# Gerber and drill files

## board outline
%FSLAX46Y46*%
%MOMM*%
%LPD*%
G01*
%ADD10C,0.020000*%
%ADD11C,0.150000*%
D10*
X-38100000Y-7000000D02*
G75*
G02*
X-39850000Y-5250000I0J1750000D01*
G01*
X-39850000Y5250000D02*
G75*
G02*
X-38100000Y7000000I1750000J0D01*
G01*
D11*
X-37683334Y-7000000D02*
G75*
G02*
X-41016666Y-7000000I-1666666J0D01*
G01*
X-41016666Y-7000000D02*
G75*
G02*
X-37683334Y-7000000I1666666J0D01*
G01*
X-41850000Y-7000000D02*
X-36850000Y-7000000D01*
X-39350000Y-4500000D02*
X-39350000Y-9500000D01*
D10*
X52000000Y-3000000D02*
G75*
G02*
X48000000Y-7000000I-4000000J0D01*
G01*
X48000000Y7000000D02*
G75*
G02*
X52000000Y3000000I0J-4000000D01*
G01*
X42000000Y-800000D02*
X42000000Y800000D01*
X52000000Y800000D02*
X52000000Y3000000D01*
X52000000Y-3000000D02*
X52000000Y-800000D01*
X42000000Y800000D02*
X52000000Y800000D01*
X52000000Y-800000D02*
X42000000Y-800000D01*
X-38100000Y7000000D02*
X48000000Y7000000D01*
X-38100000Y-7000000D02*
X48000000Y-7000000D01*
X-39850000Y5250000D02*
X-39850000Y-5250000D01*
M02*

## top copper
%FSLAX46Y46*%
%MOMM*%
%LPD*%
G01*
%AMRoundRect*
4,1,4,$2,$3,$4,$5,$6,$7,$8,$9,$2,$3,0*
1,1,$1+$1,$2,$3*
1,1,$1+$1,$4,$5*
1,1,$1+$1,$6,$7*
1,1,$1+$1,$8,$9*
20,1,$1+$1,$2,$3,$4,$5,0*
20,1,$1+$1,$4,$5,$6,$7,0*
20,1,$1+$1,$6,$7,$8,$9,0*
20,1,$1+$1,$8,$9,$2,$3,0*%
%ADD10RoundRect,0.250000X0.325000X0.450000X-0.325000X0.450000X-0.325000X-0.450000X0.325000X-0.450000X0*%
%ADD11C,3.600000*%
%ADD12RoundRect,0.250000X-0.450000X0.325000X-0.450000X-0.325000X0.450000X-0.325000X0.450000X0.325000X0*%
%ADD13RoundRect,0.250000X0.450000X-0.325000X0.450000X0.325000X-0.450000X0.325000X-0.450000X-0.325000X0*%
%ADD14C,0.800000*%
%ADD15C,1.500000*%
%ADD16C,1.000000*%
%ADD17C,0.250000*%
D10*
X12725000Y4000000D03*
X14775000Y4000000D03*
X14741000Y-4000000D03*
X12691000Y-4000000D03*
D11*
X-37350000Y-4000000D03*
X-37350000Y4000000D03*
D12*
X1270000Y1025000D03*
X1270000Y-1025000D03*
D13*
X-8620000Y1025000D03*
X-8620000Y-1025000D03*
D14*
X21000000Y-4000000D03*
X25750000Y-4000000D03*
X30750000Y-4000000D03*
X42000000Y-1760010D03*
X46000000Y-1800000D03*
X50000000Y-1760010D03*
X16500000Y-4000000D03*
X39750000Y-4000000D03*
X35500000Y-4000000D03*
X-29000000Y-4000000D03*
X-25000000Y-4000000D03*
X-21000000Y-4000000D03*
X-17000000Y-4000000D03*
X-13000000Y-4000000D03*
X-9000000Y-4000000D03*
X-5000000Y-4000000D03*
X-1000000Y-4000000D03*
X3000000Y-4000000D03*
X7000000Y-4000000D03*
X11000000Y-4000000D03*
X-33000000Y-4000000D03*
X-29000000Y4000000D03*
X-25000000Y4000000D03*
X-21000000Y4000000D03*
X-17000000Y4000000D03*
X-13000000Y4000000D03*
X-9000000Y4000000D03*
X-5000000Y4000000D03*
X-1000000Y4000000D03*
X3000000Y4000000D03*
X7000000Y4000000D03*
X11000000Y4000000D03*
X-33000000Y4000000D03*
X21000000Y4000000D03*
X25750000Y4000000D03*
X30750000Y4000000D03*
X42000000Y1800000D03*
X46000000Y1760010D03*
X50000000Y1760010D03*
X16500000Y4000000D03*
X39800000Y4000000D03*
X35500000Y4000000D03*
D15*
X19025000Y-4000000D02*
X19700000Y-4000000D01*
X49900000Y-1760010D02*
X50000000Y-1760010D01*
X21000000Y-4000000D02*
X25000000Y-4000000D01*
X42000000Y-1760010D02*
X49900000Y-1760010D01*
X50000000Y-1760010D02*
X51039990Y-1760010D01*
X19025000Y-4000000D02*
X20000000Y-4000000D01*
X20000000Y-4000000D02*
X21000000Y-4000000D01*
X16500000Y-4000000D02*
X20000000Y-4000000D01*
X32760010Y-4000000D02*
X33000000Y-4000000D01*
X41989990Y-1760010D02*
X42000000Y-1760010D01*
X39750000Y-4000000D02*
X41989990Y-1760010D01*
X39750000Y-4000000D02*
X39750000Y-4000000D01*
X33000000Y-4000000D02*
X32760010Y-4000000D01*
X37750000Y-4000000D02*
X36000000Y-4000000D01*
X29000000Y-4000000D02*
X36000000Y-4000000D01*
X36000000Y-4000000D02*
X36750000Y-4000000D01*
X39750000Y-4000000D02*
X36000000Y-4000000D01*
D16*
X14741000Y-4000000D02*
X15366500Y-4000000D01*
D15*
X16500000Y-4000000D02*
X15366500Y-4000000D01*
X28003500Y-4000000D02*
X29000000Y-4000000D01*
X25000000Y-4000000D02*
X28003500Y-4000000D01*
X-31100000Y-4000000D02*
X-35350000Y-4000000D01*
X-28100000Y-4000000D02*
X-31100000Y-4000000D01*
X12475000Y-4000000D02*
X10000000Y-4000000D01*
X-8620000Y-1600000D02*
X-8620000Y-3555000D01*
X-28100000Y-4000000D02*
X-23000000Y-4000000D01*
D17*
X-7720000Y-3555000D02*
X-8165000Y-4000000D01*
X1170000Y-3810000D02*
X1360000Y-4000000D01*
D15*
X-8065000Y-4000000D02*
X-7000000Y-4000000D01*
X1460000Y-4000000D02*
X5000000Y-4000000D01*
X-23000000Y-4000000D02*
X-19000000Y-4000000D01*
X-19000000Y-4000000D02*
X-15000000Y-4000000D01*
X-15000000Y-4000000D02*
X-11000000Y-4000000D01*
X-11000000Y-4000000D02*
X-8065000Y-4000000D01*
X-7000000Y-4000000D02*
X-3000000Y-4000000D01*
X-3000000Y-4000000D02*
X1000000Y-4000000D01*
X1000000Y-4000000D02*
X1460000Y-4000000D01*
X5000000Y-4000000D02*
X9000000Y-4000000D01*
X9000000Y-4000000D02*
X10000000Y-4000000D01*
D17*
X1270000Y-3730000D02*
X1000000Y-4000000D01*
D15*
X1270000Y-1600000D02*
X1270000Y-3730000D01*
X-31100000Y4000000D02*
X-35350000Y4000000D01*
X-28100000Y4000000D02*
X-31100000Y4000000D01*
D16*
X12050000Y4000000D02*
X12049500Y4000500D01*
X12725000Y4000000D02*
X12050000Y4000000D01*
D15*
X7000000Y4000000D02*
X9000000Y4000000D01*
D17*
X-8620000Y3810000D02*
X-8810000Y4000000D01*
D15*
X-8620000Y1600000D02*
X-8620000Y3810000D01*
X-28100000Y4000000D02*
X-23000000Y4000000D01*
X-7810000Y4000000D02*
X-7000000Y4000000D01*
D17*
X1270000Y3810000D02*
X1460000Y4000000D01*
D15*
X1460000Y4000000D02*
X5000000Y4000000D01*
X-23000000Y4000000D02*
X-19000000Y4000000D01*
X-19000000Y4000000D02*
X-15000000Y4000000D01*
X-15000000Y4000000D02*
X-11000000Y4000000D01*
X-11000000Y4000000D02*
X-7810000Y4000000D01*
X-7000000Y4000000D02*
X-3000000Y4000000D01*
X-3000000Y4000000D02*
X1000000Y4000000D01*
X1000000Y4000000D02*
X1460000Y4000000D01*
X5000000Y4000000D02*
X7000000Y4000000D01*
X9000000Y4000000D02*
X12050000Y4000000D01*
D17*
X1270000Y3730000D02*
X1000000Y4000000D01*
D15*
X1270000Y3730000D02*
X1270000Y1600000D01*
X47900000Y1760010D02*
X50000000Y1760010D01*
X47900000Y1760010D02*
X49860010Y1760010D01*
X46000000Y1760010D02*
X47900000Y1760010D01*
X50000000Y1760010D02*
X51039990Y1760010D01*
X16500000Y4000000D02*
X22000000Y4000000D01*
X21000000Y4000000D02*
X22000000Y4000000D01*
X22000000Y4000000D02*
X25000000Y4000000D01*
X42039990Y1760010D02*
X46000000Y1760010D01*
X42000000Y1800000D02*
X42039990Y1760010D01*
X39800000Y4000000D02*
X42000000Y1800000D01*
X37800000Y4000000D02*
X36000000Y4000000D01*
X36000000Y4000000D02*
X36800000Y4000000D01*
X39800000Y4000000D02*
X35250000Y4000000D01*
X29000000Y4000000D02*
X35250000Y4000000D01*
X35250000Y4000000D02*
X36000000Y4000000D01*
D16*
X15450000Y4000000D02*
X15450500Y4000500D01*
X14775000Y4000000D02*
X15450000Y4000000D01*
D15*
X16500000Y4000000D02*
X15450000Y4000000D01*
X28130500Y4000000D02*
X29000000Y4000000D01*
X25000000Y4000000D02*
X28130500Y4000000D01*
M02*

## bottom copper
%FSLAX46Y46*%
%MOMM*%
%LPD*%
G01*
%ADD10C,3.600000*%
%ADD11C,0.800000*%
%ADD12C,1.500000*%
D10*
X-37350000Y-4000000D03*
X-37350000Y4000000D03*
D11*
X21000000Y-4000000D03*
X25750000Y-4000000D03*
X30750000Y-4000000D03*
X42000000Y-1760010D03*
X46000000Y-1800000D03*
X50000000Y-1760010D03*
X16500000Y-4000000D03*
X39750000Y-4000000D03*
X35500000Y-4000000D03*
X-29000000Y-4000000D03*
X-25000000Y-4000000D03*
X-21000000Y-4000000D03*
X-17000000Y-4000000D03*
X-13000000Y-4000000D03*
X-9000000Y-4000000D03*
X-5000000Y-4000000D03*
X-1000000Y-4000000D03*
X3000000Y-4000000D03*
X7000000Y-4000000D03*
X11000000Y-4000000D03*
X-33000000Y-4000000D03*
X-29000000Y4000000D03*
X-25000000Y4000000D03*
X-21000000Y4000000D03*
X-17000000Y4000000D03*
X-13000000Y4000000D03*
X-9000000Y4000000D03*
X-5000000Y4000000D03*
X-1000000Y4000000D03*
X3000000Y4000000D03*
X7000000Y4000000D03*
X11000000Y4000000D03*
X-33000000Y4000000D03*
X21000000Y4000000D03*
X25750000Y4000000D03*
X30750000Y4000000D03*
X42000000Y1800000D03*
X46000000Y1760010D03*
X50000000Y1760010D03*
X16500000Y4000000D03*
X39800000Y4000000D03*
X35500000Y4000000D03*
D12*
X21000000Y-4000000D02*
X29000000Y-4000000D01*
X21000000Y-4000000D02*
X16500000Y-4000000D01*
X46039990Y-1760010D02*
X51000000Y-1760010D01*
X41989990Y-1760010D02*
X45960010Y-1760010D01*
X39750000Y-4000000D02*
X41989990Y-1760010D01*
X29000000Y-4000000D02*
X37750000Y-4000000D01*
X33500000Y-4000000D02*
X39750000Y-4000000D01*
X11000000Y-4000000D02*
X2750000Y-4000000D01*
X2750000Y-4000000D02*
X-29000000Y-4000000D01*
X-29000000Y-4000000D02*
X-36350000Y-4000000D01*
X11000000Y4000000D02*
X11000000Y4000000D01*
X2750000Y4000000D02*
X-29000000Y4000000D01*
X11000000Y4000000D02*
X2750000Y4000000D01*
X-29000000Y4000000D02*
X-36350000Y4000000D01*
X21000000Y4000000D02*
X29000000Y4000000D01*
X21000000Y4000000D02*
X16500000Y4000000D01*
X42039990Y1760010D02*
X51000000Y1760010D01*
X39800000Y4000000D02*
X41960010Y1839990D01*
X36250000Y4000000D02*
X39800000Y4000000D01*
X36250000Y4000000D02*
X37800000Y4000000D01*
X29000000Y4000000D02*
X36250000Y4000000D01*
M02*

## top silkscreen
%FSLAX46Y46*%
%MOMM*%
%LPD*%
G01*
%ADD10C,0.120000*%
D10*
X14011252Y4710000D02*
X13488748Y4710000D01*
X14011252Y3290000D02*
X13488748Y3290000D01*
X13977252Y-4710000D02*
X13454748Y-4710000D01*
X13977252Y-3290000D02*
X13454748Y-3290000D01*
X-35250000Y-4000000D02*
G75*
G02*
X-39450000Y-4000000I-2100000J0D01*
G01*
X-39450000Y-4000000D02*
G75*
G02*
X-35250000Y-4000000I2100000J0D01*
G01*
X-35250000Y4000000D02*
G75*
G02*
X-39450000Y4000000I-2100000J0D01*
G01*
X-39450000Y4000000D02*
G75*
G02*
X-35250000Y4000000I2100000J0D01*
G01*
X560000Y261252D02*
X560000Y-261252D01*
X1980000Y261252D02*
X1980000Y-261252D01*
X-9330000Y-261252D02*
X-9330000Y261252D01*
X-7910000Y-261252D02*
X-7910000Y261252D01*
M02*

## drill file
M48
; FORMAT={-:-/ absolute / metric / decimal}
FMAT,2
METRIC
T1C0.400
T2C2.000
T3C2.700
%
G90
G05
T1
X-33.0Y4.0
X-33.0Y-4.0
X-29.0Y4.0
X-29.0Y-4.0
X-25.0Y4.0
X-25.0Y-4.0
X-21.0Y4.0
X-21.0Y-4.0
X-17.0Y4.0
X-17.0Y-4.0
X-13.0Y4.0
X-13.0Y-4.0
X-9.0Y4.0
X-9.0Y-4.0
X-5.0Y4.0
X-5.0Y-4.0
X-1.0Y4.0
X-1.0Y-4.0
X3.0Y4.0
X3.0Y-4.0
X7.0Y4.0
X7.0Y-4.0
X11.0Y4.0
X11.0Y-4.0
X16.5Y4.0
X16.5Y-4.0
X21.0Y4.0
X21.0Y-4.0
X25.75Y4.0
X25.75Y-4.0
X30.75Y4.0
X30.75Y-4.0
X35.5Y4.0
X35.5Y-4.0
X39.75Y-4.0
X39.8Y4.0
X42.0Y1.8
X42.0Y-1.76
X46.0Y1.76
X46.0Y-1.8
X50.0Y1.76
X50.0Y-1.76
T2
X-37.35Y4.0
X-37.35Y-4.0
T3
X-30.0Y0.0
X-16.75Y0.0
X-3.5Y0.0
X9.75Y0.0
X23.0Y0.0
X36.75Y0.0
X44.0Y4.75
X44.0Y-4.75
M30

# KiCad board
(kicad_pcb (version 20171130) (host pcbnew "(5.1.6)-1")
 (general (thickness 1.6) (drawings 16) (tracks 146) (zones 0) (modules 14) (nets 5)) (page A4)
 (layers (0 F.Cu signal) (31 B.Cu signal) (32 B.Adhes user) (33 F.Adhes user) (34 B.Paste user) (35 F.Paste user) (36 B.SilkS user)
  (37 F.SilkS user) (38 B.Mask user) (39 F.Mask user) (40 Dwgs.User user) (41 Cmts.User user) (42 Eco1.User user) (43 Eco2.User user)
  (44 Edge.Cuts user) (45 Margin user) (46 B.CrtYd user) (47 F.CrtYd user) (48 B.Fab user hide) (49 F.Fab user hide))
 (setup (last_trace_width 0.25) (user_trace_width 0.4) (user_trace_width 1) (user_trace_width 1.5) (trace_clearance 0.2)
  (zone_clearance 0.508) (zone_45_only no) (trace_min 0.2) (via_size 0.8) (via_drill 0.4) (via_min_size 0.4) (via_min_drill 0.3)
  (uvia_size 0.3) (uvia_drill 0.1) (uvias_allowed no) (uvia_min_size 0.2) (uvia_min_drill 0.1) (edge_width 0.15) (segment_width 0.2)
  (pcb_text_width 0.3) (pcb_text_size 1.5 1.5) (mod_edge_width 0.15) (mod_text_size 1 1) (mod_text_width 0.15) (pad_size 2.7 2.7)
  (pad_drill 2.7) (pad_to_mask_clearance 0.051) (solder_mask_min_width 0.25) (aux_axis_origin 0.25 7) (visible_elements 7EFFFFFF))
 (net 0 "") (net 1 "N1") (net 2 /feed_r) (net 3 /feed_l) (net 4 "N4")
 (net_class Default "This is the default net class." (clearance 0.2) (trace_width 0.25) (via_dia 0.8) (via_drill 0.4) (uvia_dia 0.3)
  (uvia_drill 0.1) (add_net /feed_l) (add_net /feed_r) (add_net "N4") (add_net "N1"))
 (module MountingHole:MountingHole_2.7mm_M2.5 (layer F.Cu) (at -30 0)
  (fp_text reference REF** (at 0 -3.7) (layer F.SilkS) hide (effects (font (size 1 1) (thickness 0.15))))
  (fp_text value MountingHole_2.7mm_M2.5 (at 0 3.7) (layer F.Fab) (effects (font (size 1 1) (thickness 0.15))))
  (pad 1 np_thru_hole circle (at 0 0) (size 2.7 2.7) (drill 2.7) (layers *.Cu *.Mask)))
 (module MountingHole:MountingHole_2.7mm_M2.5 (layer F.Cu) (at -16.75 0)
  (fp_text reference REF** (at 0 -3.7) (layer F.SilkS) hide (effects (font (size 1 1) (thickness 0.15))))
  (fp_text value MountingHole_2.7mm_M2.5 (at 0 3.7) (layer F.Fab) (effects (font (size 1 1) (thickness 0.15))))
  (pad 1 np_thru_hole circle (at 0 0) (size 2.7 2.7) (drill 2.7) (layers *.Cu *.Mask)))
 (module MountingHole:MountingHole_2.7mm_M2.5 (layer F.Cu) (at -3.5 0)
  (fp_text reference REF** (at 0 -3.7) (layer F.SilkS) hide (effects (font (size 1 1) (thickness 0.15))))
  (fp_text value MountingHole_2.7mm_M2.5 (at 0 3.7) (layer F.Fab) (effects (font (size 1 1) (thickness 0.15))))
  (pad 1 np_thru_hole circle (at 0 0) (size 2.7 2.7) (drill 2.7) (layers *.Cu *.Mask)))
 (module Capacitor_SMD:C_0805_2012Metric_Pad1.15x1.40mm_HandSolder (layer F.Cu) (at 13.75 -4 180)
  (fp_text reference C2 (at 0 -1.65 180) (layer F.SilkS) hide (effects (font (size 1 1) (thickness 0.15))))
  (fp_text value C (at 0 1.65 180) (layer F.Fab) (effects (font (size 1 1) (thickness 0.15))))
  (fp_line (start -0.261252 0.71) (end 0.261252 0.71) (layer F.SilkS) (width 0.12))
  (fp_line (start -0.261252 -0.71) (end 0.261252 -0.71) (layer F.SilkS) (width 0.12))
  (pad 2 smd roundrect (at 1.025 0 180) (size 1.15 1.4) (layers F.Cu F.Paste F.Mask) (roundrect_rratio 0.217391) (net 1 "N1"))
  (pad 1 smd roundrect (at -1.025 0 180) (size 1.15 1.4) (layers F.Cu F.Paste F.Mask) (roundrect_rratio 0.217391) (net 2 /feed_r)))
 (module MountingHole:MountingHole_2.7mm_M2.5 (layer F.Cu) (at 23 0)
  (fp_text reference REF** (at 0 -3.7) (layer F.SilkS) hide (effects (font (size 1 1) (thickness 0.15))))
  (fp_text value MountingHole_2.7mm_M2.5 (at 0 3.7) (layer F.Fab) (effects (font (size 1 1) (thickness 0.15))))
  (pad 1 np_thru_hole circle (at 0 0) (size 2.7 2.7) (drill 2.7) (layers *.Cu *.Mask)))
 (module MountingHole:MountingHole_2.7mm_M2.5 (layer F.Cu) (at 44 -4.75)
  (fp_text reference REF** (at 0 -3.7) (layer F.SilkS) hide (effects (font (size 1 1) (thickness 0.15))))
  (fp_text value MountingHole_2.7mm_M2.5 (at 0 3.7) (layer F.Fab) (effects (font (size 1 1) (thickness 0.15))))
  (pad 1 np_thru_hole circle (at 0 0) (size 2.7 2.7) (drill 2.7) (layers *.Cu *.Mask)))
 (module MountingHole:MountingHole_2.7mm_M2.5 (layer F.Cu) (at 44 4.75)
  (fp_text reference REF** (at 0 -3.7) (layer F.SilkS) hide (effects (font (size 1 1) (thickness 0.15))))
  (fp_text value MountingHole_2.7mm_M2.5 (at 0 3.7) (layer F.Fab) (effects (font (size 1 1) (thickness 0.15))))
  (pad 1 np_thru_hole circle (at 0 0) (size 2.7 2.7) (drill 2.7) (layers *.Cu *.Mask)))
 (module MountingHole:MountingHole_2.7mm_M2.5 (layer F.Cu) (at 36.75 0)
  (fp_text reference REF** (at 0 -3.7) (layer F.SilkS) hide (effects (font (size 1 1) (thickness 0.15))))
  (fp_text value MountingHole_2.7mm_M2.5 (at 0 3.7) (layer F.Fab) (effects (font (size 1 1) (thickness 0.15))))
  (pad 1 np_thru_hole circle (at 0 0) (size 2.7 2.7) (drill 2.7) (layers *.Cu *.Mask)))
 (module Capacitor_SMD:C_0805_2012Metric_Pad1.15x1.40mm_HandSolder (layer F.Cu) (at 13.716 4 180)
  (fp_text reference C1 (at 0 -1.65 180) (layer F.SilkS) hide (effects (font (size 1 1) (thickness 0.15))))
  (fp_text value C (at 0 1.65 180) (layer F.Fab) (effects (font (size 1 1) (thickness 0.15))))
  (fp_line (start -0.261252 -0.71) (end 0.261252 -0.71) (layer F.SilkS) (width 0.12))
  (fp_line (start -0.261252 0.71) (end 0.261252 0.71) (layer F.SilkS) (width 0.12))
  (pad 1 smd roundrect (at -1.025 0 180) (size 1.15 1.4) (layers F.Cu F.Paste F.Mask) (roundrect_rratio 0.217391) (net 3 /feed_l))
  (pad 2 smd roundrect (at 1.025 0 180) (size 1.15 1.4) (layers F.Cu F.Paste F.Mask) (roundrect_rratio 0.217391) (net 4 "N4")))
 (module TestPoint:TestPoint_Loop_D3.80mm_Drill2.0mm (layer F.Cu) (at -37.35 4)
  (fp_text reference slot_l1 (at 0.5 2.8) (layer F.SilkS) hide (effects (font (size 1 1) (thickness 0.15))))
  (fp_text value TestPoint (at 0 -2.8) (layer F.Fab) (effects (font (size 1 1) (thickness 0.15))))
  (fp_circle (center 0 0) (end 2.1 0) (layer F.SilkS) (width 0.12))
  (pad 1 thru_hole circle (at 0 0) (size 3.6 3.6) (drill 2) (layers *.Cu *.Mask) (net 4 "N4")))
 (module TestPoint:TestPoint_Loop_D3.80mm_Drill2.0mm (layer F.Cu) (at -37.35 -4)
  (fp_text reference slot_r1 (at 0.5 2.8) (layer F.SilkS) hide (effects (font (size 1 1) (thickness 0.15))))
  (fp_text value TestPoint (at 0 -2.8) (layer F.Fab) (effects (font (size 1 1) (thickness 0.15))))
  (fp_circle (center 0 0) (end 2.1 0) (layer F.SilkS) (width 0.12))
  (pad 1 thru_hole circle (at 0 0) (size 3.6 3.6) (drill 2) (layers *.Cu *.Mask) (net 1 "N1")))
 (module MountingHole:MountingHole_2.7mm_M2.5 (layer F.Cu) (at 9.75 0)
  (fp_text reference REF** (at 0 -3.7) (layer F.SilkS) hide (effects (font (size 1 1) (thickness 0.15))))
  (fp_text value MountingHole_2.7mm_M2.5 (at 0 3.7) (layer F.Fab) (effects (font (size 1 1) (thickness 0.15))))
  (pad 1 np_thru_hole circle (at 0 0) (size 2.7 2.7) (drill 2.7) (layers *.Cu *.Mask)))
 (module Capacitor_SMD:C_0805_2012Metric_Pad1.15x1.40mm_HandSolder (layer F.Cu) (at 1.27 0 270)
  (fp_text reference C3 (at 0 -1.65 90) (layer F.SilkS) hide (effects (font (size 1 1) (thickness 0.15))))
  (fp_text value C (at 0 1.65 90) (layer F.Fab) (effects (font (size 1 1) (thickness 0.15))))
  (fp_line (start -0.261252 0.71) (end 0.261252 0.71) (layer F.SilkS) (width 0.12))
  (fp_line (start -0.261252 -0.71) (end 0.261252 -0.71) (layer F.SilkS) (width 0.12))
  (pad 1 smd roundrect (at -1.025 0 270) (size 1.15 1.4) (layers F.Cu F.Paste F.Mask) (roundrect_rratio 0.217391) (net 1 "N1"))
  (pad 2 smd roundrect (at 1.025 0 270) (size 1.15 1.4) (layers F.Cu F.Paste F.Mask) (roundrect_rratio 0.217391) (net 4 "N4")))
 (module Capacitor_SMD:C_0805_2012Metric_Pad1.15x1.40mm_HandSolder (layer F.Cu) (at -8.62 0 90)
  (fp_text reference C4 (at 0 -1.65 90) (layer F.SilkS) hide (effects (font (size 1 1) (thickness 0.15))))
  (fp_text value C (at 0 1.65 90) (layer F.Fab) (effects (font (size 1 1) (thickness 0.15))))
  (fp_line (start -0.261252 -0.71) (end 0.261252 -0.71) (layer F.SilkS) (width 0.12))
  (fp_line (start -0.261252 0.71) (end 0.261252 0.71) (layer F.SilkS) (width 0.12))
  (pad 2 smd roundrect (at 1.025 0 90) (size 1.15 1.4) (layers F.Cu F.Paste F.Mask) (roundrect_rratio 0.217391) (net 1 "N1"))
  (pad 1 smd roundrect (at -1.025 0 90) (size 1.15 1.4) (layers F.Cu F.Paste F.Mask) (roundrect_rratio 0.217391) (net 4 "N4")))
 (gr_arc (start -38.1 5.25) (end -39.85 5.25) (angle -90) (layer Edge.Cuts) (width 0.02))
 (gr_arc (start -38.1 -5.25) (end -38.1 -7) (angle -90) (layer Edge.Cuts) (width 0.02))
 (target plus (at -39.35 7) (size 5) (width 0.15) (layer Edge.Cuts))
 (gr_arc (start 48 3) (end 48 7) (angle -90) (layer Edge.Cuts) (width 0.02))
 (gr_arc (start 48 -3) (end 52 -3) (angle -90) (layer Edge.Cuts) (width 0.02))
 (gr_line (start 42 0.8) (end 42 -0.8) (layer Edge.Cuts) (width 0.02))
 (gr_line (start 52 -0.8) (end 52 -3) (layer Edge.Cuts) (width 0.02))
 (gr_line (start 52 3) (end 52 0.8) (layer Edge.Cuts) (width 0.02))
 (gr_line (start 42 -0.8) (end 52 -0.8) (layer Edge.Cuts) (width 0.02))
 (gr_line (start 52 0.8) (end 42 0.8) (layer Edge.Cuts) (width 0.02))
 (gr_line (start -38.1 -7) (end 48 -7) (layer Edge.Cuts) (width 0.02))
 (gr_line (start -38.1 7) (end 48 7) (layer Edge.Cuts) (width 0.02))
 (gr_line (start -39.85 -5.25) (end -39.85 5.25) (layer Edge.Cuts) (width 0.02))
 (segment (start 19.025 4) (end 19.7 4) (width 1.5) (layer F.Cu) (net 3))
 (segment (start 49.9 1.76001) (end 50 1.76001) (width 1.5) (layer F.Cu) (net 3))
 (segment (start 21 4) (end 25 4) (width 1.5) (layer F.Cu) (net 3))
 (via (at 21 4) (size 0.8) (drill 0.4) (layers F.Cu B.Cu) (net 3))
 (segment (start 21 4) (end 29 4) (width 1.5) (layer B.Cu) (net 3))
 (via (at 25.75 4) (size 0.8) (drill 0.4) (layers F.Cu B.Cu) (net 3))
 (via (at 30.75 4) (size 0.8) (drill 0.4) (layers F.Cu B.Cu) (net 3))
 (segment (start 42 1.76001) (end 49.9 1.76001) (width 1.5) (layer F.Cu) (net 3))
 (via (at 42 1.76001) (size 0.8) (drill 0.4) (layers F.Cu B.Cu) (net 3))
 (via (at 46 1.8) (size 0.8) (drill 0.4) (layers F.Cu B.Cu) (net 3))
 (via (at 50 1.76001) (size 0.8) (drill 0.4) (layers F.Cu B.Cu) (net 3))
 (segment (start 50 1.76001) (end 51.03999 1.76001) (width 1.5) (layer F.Cu) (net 3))
 (segment (start 19.025 4) (end 20 4) (width 1.5) (layer F.Cu) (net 3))
 (segment (start 20 4) (end 21 4) (width 1.5) (layer F.Cu) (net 3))
 (segment (start 16.5 4) (end 20 4) (width 1.5) (layer F.Cu) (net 3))
 (via (at 16.5 4) (size 0.8) (drill 0.4) (layers F.Cu B.Cu) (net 3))
 (segment (start 21 4) (end 16.5 4) (width 1.5) (layer B.Cu) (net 3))
 (segment (start 32.76001 4) (end 33 4) (width 1.5) (layer F.Cu) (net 3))
 (segment (start 46.03999 1.76001) (end 51 1.76001) (width 1.5) (layer B.Cu) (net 3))
 (segment (start 41.98999 1.76001) (end 42 1.76001) (width 1.5) (layer F.Cu) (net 3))
 (segment (start 39.75 4) (end 41.98999 1.76001) (width 1.5) (layer F.Cu) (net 3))
 (segment (start 41.98999 1.76001) (end 45.96001 1.76001) (width 1.5) (layer B.Cu) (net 3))
 (segment (start 39.75 4) (end 41.98999 1.76001) (width 1.5) (layer B.Cu) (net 3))
 (segment (start 39.75 4) (end 39.75 4) (width 1.5) (layer F.Cu) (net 3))
 (via (at 39.75 4) (size 0.8) (drill 0.4) (layers F.Cu B.Cu) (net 3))
 (segment (start 33 4) (end 32.76001 4) (width 1.5) (layer F.Cu) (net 3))
 (via (at 35.5 4) (size 0.8) (drill 0.4) (layers F.Cu B.Cu) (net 3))
 (segment (start 37.75 4) (end 36 4) (width 1.5) (layer F.Cu) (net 3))
 (segment (start 29 4) (end 36 4) (width 1.5) (layer F.Cu) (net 3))
 (segment (start 36 4) (end 36.75 4) (width 1.5) (layer F.Cu) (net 3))
 (segment (start 29 4) (end 37.75 4) (width 1.5) (layer B.Cu) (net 3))
 (segment (start 39.75 4) (end 36 4) (width 1.5) (layer F.Cu) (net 3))
 (segment (start 33.5 4) (end 39.75 4) (width 1.5) (layer B.Cu) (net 3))
 (segment (start 14.741 4) (end 15.3665 4) (width 1) (layer F.Cu) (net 3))
 (segment (start 16.5 4) (end 15.3665 4) (width 1.5) (layer F.Cu) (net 3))
 (segment (start 28.0035 4) (end 29 4) (width 1.5) (layer F.Cu) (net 3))
 (segment (start 25 4) (end 28.0035 4) (width 1.5) (layer F.Cu) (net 3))
 (segment (start -31.1 4) (end -35.35 4) (width 1.5) (layer F.Cu) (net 4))
 (via (at -29 4) (size 0.8) (drill 0.4) (layers F.Cu B.Cu) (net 4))
 (segment (start -28.1 4) (end -31.1 4) (width 1.5) (layer F.Cu) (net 4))
 (via (at -25 4) (size 0.8) (drill 0.4) (layers F.Cu B.Cu) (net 4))
 (segment (start 11 4) (end 2.75 4) (width 1.5) (layer B.Cu) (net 4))
 (segment (start 12.475 4) (end 10 4) (width 1.5) (layer F.Cu) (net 4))
 (segment (start -8.62 1.6) (end -8.62 3.555) (width 1.5) (layer F.Cu) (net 4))
 (segment (start -28.1 4) (end -23 4) (width 1.5) (layer F.Cu) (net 4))
 (segment (start -7.72 3.555) (end -8.165 4) (width 0.25) (layer F.Cu) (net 4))
 (segment (start 1.17 3.81) (end 1.36 4) (width 0.25) (layer F.Cu) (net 4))
 (segment (start -8.065 4) (end -7 4) (width 1.5) (layer F.Cu) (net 4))
 (segment (start 1.46 4) (end 5 4) (width 1.5) (layer F.Cu) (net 4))
 (segment (start -23 4) (end -19 4) (width 1.5) (layer F.Cu) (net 4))
 (via (at -21 4) (size 0.8) (drill 0.4) (layers F.Cu B.Cu) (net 4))
 (segment (start -19 4) (end -15 4) (width 1.5) (layer F.Cu) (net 4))
 (via (at -17 4) (size 0.8) (drill 0.4) (layers F.Cu B.Cu) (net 4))
 (segment (start -15 4) (end -11 4) (width 1.5) (layer F.Cu) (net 4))
 (via (at -13 4) (size 0.8) (drill 0.4) (layers F.Cu B.Cu) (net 4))
 (segment (start -11 4) (end -8.065 4) (width 1.5) (layer F.Cu) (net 4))
 (via (at -9 4) (size 0.8) (drill 0.4) (layers F.Cu B.Cu) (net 4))
 (segment (start -7 4) (end -3 4) (width 1.5) (layer F.Cu) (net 4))
 (via (at -5 4) (size 0.8) (drill 0.4) (layers F.Cu B.Cu) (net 4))
 (segment (start -3 4) (end 1 4) (width 1.5) (layer F.Cu) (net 4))
 (via (at -1 4) (size 0.8) (drill 0.4) (layers F.Cu B.Cu) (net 4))
 (segment (start 1 4) (end 1.46 4) (width 1.5) (layer F.Cu) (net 4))
 (via (at 3 4) (size 0.8) (drill 0.4) (layers F.Cu B.Cu) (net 4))
 (segment (start 5 4) (end 9 4) (width 1.5) (layer F.Cu) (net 4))
 (via (at 7 4) (size 0.8) (drill 0.4) (layers F.Cu B.Cu) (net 4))
 (segment (start 9 4) (end 10 4) (width 1.5) (layer F.Cu) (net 4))
 (via (at 11 4) (size 0.8) (drill 0.4) (layers F.Cu B.Cu) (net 4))
 (segment (start 1.27 3.73) (end 1 4) (width 0.25) (layer F.Cu) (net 4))
 (segment (start 1.27 1.6) (end 1.27 3.73) (width 1.5) (layer F.Cu) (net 4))
 (segment (start 2.75 4) (end -29 4) (width 1.5) (layer B.Cu) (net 4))
 (segment (start -29 4) (end -36.35 4) (width 1.5) (layer B.Cu) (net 4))
 (via (at -33 4) (size 0.8) (drill 0.4) (layers F.Cu B.Cu) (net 4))
 (segment (start -31.1 -4) (end -35.35 -4) (width 1.5) (layer F.Cu) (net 1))
 (via (at -29 -4) (size 0.8) (drill 0.4) (layers F.Cu B.Cu) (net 1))
 (segment (start -28.1 -4) (end -31.1 -4) (width 1.5) (layer F.Cu) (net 1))
 (via (at -25 -4) (size 0.8) (drill 0.4) (layers F.Cu B.Cu) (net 1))
 (segment (start 11 -4) (end 11 -4) (width 1.5) (layer B.Cu) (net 1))
 (segment (start 12.05 -4) (end 12.0495 -4.0005) (width 1) (layer F.Cu) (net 1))
 (segment (start 12.725 -4) (end 12.05 -4) (width 1) (layer F.Cu) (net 1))
 (segment (start 7 -4) (end 9 -4) (width 1.5) (layer F.Cu) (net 1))
 (segment (start -8.62 -3.81) (end -8.81 -4) (width 0.25) (layer F.Cu) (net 1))
 (segment (start -8.62 -1.6) (end -8.62 -3.81) (width 1.5) (layer F.Cu) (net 1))
 (segment (start -28.1 -4) (end -23 -4) (width 1.5) (layer F.Cu) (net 1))
 (segment (start -7.81 -4) (end -7 -4) (width 1.5) (layer F.Cu) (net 1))
 (segment (start 1.27 -3.81) (end 1.46 -4) (width 0.25) (layer F.Cu) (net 1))
 (segment (start 1.46 -4) (end 5 -4) (width 1.5) (layer F.Cu) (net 1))
 (segment (start -23 -4) (end -19 -4) (width 1.5) (layer F.Cu) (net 1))
 (via (at -21 -4) (size 0.8) (drill 0.4) (layers F.Cu B.Cu) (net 1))
 (segment (start -19 -4) (end -15 -4) (width 1.5) (layer F.Cu) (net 1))
 (via (at -17 -4) (size 0.8) (drill 0.4) (layers F.Cu B.Cu) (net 1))
 (segment (start -15 -4) (end -11 -4) (width 1.5) (layer F.Cu) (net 1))
 (via (at -13 -4) (size 0.8) (drill 0.4) (layers F.Cu B.Cu) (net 1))
 (segment (start -11 -4) (end -7.81 -4) (width 1.5) (layer F.Cu) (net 1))
 (via (at -9 -4) (size 0.8) (drill 0.4) (layers F.Cu B.Cu) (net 1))
 (segment (start -7 -4) (end -3 -4) (width 1.5) (layer F.Cu) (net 1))
 (via (at -5 -4) (size 0.8) (drill 0.4) (layers F.Cu B.Cu) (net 1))
 (segment (start -3 -4) (end 1 -4) (width 1.5) (layer F.Cu) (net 1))
 (via (at -1 -4) (size 0.8) (drill 0.4) (layers F.Cu B.Cu) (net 1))
 (segment (start 1 -4) (end 1.46 -4) (width 1.5) (layer F.Cu) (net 1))
 (via (at 3 -4) (size 0.8) (drill 0.4) (layers F.Cu B.Cu) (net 1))
 (segment (start 5 -4) (end 7 -4) (width 1.5) (layer F.Cu) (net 1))
 (via (at 7 -4) (size 0.8) (drill 0.4) (layers F.Cu B.Cu) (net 1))
 (segment (start 9 -4) (end 12.05 -4) (width 1.5) (layer F.Cu) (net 1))
 (via (at 11 -4) (size 0.8) (drill 0.4) (layers F.Cu B.Cu) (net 1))
 (segment (start 1.27 -3.73) (end 1 -4) (width 0.25) (layer F.Cu) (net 1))
 (segment (start 1.27 -3.73) (end 1.27 -1.6) (width 1.5) (layer F.Cu) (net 1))
 (segment (start 2.75 -4) (end -29 -4) (width 1.5) (layer B.Cu) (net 1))
 (segment (start 11 -4) (end 2.75 -4) (width 1.5) (layer B.Cu) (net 1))
 (segment (start -29 -4) (end -36.35 -4) (width 1.5) (layer B.Cu) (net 1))
 (via (at -33 -4) (size 0.8) (drill 0.4) (layers F.Cu B.Cu) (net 1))
 (segment (start 47.9 -1.76001) (end 50 -1.76001) (width 1.5) (layer F.Cu) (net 2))
 (segment (start 47.9 -1.76001) (end 49.86001 -1.76001) (width 1.5) (layer F.Cu) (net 2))
 (via (at 21 -4) (size 0.8) (drill 0.4) (layers F.Cu B.Cu) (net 2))
 (segment (start 21 -4) (end 29 -4) (width 1.5) (layer B.Cu) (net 2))
 (via (at 25.75 -4) (size 0.8) (drill 0.4) (layers F.Cu B.Cu) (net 2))
 (via (at 30.75 -4) (size 0.8) (drill 0.4) (layers F.Cu B.Cu) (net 2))
 (via (at 42 -1.8) (size 0.8) (drill 0.4) (layers F.Cu B.Cu) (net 2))
 (segment (start 46 -1.76001) (end 47.9 -1.76001) (width 1.5) (layer F.Cu) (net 2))
 (via (at 46 -1.76001) (size 0.8) (drill 0.4) (layers F.Cu B.Cu) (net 2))
 (via (at 50 -1.76001) (size 0.8) (drill 0.4) (layers F.Cu B.Cu) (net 2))
 (segment (start 50 -1.76001) (end 51.03999 -1.76001) (width 1.5) (layer F.Cu) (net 2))
 (via (at 16.5 -4) (size 0.8) (drill 0.4) (layers F.Cu B.Cu) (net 2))
 (segment (start 21 -4) (end 16.5 -4) (width 1.5) (layer B.Cu) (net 2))
 (segment (start 42.03999 -1.76001) (end 51 -1.76001) (width 1.5) (layer B.Cu) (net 2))
 (segment (start 16.5 -4) (end 22 -4) (width 1.5) (layer F.Cu) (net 2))
 (segment (start 21 -4) (end 22 -4) (width 1.5) (layer F.Cu) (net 2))
 (segment (start 22 -4) (end 25 -4) (width 1.5) (layer F.Cu) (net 2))
 (segment (start 42.03999 -1.76001) (end 46 -1.76001) (width 1.5) (layer F.Cu) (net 2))
 (segment (start 42 -1.8) (end 42.03999 -1.76001) (width 1.5) (layer F.Cu) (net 2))
 (segment (start 39.8 -4) (end 41.96001 -1.83999) (width 1.5) (layer B.Cu) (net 2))
 (segment (start 39.8 -4) (end 42 -1.8) (width 1.5) (layer F.Cu) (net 2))
 (via (at 39.8 -4) (size 0.8) (drill 0.4) (layers F.Cu B.Cu) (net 2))
 (via (at 35.5 -4) (size 0.8) (drill 0.4) (layers F.Cu B.Cu) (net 2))
 (segment (start 37.8 -4) (end 36 -4) (width 1.5) (layer F.Cu) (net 2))
 (segment (start 36 -4) (end 36.8 -4) (width 1.5) (layer F.Cu) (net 2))
 (segment (start 39.8 -4) (end 35.25 -4) (width 1.5) (layer F.Cu) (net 2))
 (segment (start 29 -4) (end 35.25 -4) (width 1.5) (layer F.Cu) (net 2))
 (segment (start 35.25 -4) (end 36 -4) (width 1.5) (layer F.Cu) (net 2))
 (segment (start 36.25 -4) (end 39.8 -4) (width 1.5) (layer B.Cu) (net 2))
 (segment (start 36.25 -4) (end 37.8 -4) (width 1.5) (layer B.Cu) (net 2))
 (segment (start 29 -4) (end 36.25 -4) (width 1.5) (layer B.Cu) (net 2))
 (segment (start 15.45 -4) (end 15.4505 -4.0005) (width 1) (layer F.Cu) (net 2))
 (segment (start 14.775 -4) (end 15.45 -4) (width 1) (layer F.Cu) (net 2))
 (segment (start 16.5 -4) (end 15.45 -4) (width 1.5) (layer F.Cu) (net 2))
 (segment (start 28.1305 -4) (end 29 -4) (width 1.5) (layer F.Cu) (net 2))
 (segment (start 25 -4) (end 28.1305 -4) (width 1.5) (layer F.Cu) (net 2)))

